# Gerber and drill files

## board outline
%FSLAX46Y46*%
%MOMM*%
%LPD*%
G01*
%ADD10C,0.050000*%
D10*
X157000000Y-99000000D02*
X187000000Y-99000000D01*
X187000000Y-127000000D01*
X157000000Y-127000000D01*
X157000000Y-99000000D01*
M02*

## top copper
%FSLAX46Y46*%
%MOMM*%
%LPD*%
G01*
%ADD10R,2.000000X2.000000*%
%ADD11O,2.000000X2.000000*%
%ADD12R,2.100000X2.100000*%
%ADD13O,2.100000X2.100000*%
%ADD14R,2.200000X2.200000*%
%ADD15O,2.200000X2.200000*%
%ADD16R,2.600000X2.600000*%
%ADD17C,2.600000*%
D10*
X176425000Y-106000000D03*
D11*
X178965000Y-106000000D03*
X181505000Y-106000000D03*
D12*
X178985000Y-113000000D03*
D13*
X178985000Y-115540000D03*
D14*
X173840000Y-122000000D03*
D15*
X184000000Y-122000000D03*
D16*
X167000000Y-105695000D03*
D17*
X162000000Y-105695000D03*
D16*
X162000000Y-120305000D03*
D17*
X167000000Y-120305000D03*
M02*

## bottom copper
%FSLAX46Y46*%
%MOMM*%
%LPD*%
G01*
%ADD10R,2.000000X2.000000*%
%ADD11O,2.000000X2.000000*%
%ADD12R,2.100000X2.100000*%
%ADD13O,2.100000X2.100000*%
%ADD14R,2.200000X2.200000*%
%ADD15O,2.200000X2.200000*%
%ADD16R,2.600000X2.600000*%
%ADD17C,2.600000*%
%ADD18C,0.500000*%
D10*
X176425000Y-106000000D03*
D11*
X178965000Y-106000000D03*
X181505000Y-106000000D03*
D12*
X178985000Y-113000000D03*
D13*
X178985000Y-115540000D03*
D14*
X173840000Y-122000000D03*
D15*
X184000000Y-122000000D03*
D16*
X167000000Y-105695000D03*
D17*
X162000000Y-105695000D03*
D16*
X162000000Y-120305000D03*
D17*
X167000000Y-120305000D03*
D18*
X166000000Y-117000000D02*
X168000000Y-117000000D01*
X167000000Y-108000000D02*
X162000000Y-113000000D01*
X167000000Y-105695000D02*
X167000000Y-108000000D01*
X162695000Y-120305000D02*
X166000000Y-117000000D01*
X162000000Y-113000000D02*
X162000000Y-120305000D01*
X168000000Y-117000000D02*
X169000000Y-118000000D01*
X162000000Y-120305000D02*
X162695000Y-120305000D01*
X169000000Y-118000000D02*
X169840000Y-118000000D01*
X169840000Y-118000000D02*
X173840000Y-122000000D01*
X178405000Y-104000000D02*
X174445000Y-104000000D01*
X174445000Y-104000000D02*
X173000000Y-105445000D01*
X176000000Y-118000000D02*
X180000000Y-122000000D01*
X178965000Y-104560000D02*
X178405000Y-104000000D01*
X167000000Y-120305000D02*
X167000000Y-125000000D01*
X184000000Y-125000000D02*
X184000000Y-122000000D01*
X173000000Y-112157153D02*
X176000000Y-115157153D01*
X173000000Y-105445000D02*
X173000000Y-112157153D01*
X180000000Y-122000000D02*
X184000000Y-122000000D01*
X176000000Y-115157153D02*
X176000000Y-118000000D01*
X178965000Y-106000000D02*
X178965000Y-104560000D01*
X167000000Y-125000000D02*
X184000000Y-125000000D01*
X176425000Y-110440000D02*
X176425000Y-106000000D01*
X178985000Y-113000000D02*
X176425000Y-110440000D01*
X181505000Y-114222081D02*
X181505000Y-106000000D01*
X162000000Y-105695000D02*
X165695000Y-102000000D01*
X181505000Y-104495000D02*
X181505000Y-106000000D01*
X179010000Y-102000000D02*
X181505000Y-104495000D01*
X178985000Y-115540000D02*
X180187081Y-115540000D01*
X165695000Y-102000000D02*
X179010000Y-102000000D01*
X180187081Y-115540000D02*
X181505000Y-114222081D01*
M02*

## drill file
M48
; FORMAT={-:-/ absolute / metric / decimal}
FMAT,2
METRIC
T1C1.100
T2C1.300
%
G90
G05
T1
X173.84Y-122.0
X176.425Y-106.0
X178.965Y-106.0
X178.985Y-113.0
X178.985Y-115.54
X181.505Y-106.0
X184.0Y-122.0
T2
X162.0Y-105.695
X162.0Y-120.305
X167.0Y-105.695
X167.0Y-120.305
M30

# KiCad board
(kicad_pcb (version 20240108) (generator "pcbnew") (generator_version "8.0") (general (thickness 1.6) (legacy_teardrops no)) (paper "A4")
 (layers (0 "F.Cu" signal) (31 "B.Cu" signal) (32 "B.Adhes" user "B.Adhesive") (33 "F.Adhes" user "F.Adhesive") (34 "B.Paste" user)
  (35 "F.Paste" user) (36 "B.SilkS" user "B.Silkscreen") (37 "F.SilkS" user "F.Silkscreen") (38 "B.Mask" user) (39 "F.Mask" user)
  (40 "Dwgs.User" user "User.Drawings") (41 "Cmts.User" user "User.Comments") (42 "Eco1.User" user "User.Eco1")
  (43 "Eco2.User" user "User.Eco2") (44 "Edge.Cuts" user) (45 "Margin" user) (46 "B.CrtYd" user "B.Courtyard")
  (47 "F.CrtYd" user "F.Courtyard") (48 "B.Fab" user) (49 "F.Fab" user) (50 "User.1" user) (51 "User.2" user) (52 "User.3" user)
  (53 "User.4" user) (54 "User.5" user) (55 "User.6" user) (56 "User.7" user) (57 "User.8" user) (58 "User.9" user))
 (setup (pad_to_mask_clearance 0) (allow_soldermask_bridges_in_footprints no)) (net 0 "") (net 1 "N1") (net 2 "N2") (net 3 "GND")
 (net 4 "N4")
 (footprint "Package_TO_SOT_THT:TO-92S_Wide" (layer "F.Cu") (at 176.425 106)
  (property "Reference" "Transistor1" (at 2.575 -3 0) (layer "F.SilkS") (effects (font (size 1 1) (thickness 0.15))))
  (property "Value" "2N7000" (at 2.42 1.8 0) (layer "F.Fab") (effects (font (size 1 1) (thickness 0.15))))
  (pad "1" thru_hole rect (at 0 0) (size 2 2) (drill 1.1) (layers "*.Cu" "*.Mask") (remove_unused_layers no) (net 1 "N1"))
  (pad "2" thru_hole oval (at 2.54 0) (size 2 2) (drill 1.1) (layers "*.Cu" "*.Mask") (remove_unused_layers no) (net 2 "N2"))
  (pad "3" thru_hole oval (at 5.08 0) (size 2 2) (drill 1.1) (layers "*.Cu" "*.Mask") (remove_unused_layers no) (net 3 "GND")))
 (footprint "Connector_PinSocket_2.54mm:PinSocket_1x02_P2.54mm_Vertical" (layer "F.Cu") (at 178.985 113)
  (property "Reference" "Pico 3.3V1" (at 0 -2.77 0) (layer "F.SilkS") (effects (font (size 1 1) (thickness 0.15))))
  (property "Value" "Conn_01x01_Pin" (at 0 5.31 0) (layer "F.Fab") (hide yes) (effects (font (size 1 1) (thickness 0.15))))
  (pad "1" thru_hole rect (at 0 0) (size 2.1 2.1) (drill 1.1) (layers "*.Cu" "*.Mask") (remove_unused_layers no) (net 1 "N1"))
  (pad "2" thru_hole oval (at 0 2.54) (size 2.1 2.1) (drill 1.1) (layers "*.Cu" "*.Mask") (remove_unused_layers no) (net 3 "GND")))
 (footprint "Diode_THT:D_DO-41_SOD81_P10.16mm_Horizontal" (layer "F.Cu") (at 173.84 122)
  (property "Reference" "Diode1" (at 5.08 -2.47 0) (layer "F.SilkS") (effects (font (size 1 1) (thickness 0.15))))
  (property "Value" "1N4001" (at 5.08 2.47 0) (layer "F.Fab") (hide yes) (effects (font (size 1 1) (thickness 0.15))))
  (pad "1" thru_hole rect (at 0 0) (size 2.2 2.2) (drill 1.1) (layers "*.Cu" "*.Mask") (remove_unused_layers no) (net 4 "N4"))
  (pad "2" thru_hole oval (at 10.16 0) (size 2.2 2.2) (drill 1.1) (layers "*.Cu" "*.Mask") (remove_unused_layers no) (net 2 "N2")))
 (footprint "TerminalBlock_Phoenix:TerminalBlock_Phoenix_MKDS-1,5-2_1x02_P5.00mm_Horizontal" (layer "F.Cu") (at 167 105.695 180)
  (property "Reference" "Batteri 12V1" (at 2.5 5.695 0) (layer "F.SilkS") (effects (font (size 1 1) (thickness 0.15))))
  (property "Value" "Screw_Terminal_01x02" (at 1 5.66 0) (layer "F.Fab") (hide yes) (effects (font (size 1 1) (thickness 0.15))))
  (pad "1" thru_hole rect (at 0 0 180) (size 2.6 2.6) (drill 1.3) (layers "*.Cu" "*.Mask") (remove_unused_layers no) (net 4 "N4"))
  (pad "2" thru_hole circle (at 5 0 180) (size 2.6 2.6) (drill 1.3) (layers "*.Cu" "*.Mask") (remove_unused_layers no) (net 3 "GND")))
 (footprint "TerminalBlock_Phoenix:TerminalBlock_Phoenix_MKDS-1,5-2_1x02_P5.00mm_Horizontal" (layer "F.Cu") (at 162 120.305)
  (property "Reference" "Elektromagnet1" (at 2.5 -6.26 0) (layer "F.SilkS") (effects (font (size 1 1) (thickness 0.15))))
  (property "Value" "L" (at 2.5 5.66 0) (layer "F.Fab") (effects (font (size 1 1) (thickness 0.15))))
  (pad "1" thru_hole rect (at 0 0) (size 2.6 2.6) (drill 1.3) (layers "*.Cu" "*.Mask") (remove_unused_layers no) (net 4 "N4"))
  (pad "2" thru_hole circle (at 5 0) (size 2.6 2.6) (drill 1.3) (layers "*.Cu" "*.Mask") (remove_unused_layers no) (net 2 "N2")))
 (gr_rect (start 157 99) (end 187 127) (stroke (width 0.05) (type default)) (fill none) (layer "Edge.Cuts"))
 (segment (start 166 117) (end 168 117) (width 0.5) (layer "B.Cu") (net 4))
 (segment (start 167 108) (end 162 113) (width 0.5) (layer "B.Cu") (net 4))
 (segment (start 167 105.695) (end 167 108) (width 0.5) (layer "B.Cu") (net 4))
 (segment (start 162.695 120.305) (end 166 117) (width 0.5) (layer "B.Cu") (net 4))
 (segment (start 162 113) (end 162 120.305) (width 0.5) (layer "B.Cu") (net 4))
 (segment (start 168 117) (end 169 118) (width 0.5) (layer "B.Cu") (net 4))
 (segment (start 162 120.305) (end 162.695 120.305) (width 0.5) (layer "B.Cu") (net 4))
 (segment (start 169 118) (end 169.84 118) (width 0.5) (layer "B.Cu") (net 4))
 (segment (start 169.84 118) (end 173.84 122) (width 0.5) (layer "B.Cu") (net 4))
 (segment (start 178.405 104) (end 174.445 104) (width 0.5) (layer "B.Cu") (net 2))
 (segment (start 174.445 104) (end 173 105.445) (width 0.5) (layer "B.Cu") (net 2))
 (segment (start 176 118) (end 180 122) (width 0.5) (layer "B.Cu") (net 2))
 (segment (start 178.965 104.56) (end 178.405 104) (width 0.5) (layer "B.Cu") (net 2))
 (segment (start 167 120.305) (end 167 125) (width 0.5) (layer "B.Cu") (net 2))
 (segment (start 184 125) (end 184 122) (width 0.5) (layer "B.Cu") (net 2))
 (segment (start 173 112.157153) (end 176 115.157153) (width 0.5) (layer "B.Cu") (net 2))
 (segment (start 173 105.445) (end 173 112.157153) (width 0.5) (layer "B.Cu") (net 2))
 (segment (start 180 122) (end 184 122) (width 0.5) (layer "B.Cu") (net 2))
 (segment (start 176 115.157153) (end 176 118) (width 0.5) (layer "B.Cu") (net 2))
 (segment (start 178.965 106) (end 178.965 104.56) (width 0.5) (layer "B.Cu") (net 2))
 (segment (start 167 125) (end 184 125) (width 0.5) (layer "B.Cu") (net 2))
 (segment (start 176.425 110.44) (end 176.425 106) (width 0.5) (layer "B.Cu") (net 1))
 (segment (start 178.985 113) (end 176.425 110.44) (width 0.5) (layer "B.Cu") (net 1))
 (segment (start 181.505 114.222081) (end 181.505 106) (width 0.5) (layer "B.Cu") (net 3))
 (segment (start 162 105.695) (end 165.695 102) (width 0.5) (layer "B.Cu") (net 3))
 (segment (start 181.505 104.495) (end 181.505 106) (width 0.5) (layer "B.Cu") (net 3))
 (segment (start 179.01 102) (end 181.505 104.495) (width 0.5) (layer "B.Cu") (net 3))
 (segment (start 178.985 115.54) (end 180.187081 115.54) (width 0.5) (layer "B.Cu") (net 3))
 (segment (start 165.695 102) (end 179.01 102) (width 0.5) (layer "B.Cu") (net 3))
 (segment (start 180.187081 115.54) (end 181.505 114.222081) (width 0.5) (layer "B.Cu") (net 3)))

